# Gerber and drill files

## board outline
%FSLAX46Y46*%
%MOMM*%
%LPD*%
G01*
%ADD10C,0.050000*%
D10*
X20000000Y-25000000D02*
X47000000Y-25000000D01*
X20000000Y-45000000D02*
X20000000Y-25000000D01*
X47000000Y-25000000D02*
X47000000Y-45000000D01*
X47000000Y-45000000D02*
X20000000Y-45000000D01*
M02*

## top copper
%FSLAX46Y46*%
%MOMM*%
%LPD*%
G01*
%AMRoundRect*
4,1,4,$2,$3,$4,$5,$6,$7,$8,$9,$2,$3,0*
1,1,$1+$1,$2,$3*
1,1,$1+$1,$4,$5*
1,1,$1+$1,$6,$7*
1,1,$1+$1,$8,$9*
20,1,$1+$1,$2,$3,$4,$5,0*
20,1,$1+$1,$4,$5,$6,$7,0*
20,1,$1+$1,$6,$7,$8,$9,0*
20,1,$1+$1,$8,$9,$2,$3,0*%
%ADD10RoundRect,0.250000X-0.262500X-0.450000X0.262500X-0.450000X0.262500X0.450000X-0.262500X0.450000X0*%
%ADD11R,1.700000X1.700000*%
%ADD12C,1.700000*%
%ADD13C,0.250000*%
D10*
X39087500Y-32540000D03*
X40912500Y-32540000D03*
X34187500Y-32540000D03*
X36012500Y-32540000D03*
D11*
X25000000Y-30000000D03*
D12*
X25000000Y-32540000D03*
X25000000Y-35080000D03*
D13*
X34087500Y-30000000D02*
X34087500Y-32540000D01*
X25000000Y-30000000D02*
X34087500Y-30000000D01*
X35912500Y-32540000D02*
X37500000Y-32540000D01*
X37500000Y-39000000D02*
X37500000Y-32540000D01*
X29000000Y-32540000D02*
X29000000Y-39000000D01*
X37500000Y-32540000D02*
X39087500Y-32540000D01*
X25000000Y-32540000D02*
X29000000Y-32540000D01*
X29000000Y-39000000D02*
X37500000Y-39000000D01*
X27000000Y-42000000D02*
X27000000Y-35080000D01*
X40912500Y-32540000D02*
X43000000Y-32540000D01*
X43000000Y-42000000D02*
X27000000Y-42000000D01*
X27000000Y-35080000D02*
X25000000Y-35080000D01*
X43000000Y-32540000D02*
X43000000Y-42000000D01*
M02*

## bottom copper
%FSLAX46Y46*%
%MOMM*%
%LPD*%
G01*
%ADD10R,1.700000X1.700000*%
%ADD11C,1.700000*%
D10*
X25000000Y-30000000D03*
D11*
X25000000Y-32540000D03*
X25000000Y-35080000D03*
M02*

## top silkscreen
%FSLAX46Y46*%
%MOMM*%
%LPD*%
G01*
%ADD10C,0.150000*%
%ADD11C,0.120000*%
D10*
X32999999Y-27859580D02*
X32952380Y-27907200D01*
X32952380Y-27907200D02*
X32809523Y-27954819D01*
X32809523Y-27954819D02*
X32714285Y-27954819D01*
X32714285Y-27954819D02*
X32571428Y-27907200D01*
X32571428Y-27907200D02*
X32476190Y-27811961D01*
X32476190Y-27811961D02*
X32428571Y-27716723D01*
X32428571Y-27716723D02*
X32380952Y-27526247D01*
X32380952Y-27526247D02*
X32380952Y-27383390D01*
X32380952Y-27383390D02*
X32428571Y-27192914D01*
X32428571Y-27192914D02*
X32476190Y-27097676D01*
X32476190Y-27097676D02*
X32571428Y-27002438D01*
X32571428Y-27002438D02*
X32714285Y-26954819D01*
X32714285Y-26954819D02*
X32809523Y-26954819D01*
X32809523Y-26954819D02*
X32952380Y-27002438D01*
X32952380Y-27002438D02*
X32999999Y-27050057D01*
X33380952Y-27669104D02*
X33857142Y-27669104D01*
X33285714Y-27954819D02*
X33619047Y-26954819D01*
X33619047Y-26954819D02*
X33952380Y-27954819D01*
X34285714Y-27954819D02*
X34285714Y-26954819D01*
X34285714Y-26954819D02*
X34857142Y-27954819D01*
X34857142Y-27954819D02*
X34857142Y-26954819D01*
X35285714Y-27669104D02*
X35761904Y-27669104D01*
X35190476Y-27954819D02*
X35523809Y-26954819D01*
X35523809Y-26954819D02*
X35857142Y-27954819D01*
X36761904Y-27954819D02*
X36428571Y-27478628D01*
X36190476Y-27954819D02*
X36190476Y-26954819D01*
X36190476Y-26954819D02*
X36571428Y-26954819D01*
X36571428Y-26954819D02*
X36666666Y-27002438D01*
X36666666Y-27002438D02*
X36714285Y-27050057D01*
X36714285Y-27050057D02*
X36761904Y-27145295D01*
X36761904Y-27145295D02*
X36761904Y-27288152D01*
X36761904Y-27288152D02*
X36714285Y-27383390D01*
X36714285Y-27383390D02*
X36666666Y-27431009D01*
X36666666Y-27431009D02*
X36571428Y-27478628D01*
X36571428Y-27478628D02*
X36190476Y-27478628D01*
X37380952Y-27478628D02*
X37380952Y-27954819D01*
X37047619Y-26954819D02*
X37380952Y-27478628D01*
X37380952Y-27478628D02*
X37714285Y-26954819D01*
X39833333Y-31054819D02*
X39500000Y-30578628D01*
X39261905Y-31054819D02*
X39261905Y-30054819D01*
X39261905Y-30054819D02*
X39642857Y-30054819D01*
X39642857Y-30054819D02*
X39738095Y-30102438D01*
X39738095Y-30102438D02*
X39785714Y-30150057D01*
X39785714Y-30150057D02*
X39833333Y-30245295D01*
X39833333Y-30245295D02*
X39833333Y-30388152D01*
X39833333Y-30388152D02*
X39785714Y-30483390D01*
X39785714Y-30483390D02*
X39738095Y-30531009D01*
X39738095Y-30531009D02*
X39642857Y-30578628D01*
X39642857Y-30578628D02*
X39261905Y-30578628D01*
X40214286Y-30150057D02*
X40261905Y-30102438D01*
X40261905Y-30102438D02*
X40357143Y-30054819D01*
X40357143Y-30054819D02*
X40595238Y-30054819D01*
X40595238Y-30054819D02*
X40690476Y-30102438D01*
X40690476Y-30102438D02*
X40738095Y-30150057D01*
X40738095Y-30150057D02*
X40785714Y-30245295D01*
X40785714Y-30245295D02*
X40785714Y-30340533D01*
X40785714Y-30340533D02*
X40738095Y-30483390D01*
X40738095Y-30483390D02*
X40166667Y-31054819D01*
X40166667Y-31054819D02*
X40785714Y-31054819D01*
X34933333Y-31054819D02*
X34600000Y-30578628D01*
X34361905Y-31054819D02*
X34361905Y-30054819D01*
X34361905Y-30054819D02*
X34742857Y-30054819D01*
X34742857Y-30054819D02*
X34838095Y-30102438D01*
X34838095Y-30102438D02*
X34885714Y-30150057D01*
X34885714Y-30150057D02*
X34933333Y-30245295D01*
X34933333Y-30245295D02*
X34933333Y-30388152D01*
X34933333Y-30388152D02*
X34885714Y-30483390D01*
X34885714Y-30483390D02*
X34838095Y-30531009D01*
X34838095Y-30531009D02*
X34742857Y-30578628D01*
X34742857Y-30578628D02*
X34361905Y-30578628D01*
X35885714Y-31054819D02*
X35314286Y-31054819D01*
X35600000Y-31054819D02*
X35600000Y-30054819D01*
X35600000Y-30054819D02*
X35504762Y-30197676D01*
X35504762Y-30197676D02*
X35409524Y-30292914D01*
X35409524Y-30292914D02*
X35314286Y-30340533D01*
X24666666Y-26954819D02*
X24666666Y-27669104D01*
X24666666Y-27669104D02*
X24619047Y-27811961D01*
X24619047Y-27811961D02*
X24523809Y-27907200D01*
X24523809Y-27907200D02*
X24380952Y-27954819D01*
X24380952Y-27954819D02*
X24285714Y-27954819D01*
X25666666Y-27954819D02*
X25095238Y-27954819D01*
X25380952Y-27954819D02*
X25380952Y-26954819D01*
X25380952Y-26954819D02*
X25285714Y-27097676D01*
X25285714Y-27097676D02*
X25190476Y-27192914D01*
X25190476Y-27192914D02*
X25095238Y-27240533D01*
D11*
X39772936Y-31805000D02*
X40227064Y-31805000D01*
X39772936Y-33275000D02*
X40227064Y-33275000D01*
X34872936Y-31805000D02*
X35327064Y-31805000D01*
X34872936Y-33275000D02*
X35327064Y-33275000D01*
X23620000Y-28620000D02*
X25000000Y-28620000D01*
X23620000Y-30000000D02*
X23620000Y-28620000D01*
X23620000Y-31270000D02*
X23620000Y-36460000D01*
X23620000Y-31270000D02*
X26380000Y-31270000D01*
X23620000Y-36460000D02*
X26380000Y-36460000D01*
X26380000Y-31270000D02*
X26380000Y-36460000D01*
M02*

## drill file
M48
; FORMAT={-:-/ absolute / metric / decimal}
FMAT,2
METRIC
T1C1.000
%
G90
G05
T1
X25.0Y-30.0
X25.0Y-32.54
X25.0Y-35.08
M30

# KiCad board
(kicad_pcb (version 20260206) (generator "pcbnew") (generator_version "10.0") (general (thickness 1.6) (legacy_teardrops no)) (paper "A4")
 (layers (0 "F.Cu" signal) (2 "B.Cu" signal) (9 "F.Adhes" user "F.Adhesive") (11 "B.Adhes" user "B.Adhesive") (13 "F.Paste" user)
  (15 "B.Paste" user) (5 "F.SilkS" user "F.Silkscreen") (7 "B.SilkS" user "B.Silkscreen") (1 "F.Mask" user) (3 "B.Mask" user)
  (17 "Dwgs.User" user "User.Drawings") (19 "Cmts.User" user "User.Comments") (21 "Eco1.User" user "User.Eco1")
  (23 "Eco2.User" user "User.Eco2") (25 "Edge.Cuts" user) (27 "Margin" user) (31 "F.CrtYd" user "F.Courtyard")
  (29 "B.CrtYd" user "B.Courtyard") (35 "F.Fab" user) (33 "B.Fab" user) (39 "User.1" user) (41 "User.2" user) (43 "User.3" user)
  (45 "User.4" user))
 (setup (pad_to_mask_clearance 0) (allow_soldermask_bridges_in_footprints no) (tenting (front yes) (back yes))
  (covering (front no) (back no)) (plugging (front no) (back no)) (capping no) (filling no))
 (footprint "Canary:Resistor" (layer "F.Cu") (at 40 32.54)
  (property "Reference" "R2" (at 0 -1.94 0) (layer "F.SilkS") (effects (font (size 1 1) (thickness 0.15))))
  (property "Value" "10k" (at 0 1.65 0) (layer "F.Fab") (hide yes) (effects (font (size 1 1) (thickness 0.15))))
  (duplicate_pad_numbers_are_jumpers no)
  (fp_line (start -0.227064 -0.735) (end 0.227064 -0.735) (stroke (width 0.12) (type solid)) (layer "F.SilkS"))
  (fp_line (start -0.227064 0.735) (end 0.227064 0.735) (stroke (width 0.12) (type solid)) (layer "F.SilkS"))
  (pad "1" smd roundrect (at -0.9125 0) (size 1.025 1.4) (layers "F.Cu" "F.Mask" "F.Paste") (roundrect_rratio 0.243902) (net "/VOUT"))
  (pad "2" smd roundrect (at 0.9125 0) (size 1.025 1.4) (layers "F.Cu" "F.Mask" "F.Paste") (roundrect_rratio 0.243902) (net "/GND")))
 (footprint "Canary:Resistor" (layer "F.Cu") (at 35.1 32.54)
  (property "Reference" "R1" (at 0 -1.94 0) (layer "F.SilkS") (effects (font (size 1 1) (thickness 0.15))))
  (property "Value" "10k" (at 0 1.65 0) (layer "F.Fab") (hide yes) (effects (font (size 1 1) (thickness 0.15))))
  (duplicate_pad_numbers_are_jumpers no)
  (fp_line (start -0.227064 -0.735) (end 0.227064 -0.735) (stroke (width 0.12) (type solid)) (layer "F.SilkS"))
  (fp_line (start -0.227064 0.735) (end 0.227064 0.735) (stroke (width 0.12) (type solid)) (layer "F.SilkS"))
  (pad "1" smd roundrect (at -0.9125 0) (size 1.025 1.4) (layers "F.Cu" "F.Mask" "F.Paste") (roundrect_rratio 0.243902) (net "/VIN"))
  (pad "2" smd roundrect (at 0.9125 0) (size 1.025 1.4) (layers "F.Cu" "F.Mask" "F.Paste") (roundrect_rratio 0.243902) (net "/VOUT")))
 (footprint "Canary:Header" (layer "F.Cu") (at 25 30)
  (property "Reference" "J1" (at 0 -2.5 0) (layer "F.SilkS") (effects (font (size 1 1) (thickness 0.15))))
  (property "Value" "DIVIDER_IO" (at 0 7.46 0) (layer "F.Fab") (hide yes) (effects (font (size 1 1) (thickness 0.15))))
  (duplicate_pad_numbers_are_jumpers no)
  (fp_line (start -1.38 -1.38) (end 0 -1.38) (stroke (width 0.12) (type solid)) (layer "F.SilkS"))
  (fp_line (start -1.38 0) (end -1.38 -1.38) (stroke (width 0.12) (type solid)) (layer "F.SilkS"))
  (fp_line (start -1.38 1.27) (end -1.38 6.46) (stroke (width 0.12) (type solid)) (layer "F.SilkS"))
  (fp_line (start -1.38 1.27) (end 1.38 1.27) (stroke (width 0.12) (type solid)) (layer "F.SilkS"))
  (fp_line (start -1.38 6.46) (end 1.38 6.46) (stroke (width 0.12) (type solid)) (layer "F.SilkS"))
  (fp_line (start 1.38 1.27) (end 1.38 6.46) (stroke (width 0.12) (type solid)) (layer "F.SilkS"))
  (pad "1" thru_hole rect (at 0 0) (size 1.7 1.7) (drill 1) (layers "*.Cu" "*.Mask") (remove_unused_layers no) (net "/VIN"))
  (pad "2" thru_hole circle (at 0 2.54) (size 1.7 1.7) (drill 1) (layers "*.Cu" "*.Mask") (remove_unused_layers no) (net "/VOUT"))
  (pad "3" thru_hole circle (at 0 5.08) (size 1.7 1.7) (drill 1) (layers "*.Cu" "*.Mask") (remove_unused_layers no) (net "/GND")))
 (gr_line (start 20 25) (end 47 25) (stroke (width 0.05) (type default)) (layer "Edge.Cuts"))
 (gr_line (start 20 45) (end 20 25) (stroke (width 0.05) (type default)) (layer "Edge.Cuts"))
 (gr_line (start 47 25) (end 47 45) (stroke (width 0.05) (type default)) (layer "Edge.Cuts"))
 (gr_line (start 47 45) (end 20 45) (stroke (width 0.05) (type default)) (layer "Edge.Cuts"))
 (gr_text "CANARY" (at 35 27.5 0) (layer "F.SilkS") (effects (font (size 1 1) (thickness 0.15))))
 (segment (start 34.0875 30) (end 34.0875 32.54) (width 0.25) (layer "F.Cu") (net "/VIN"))
 (segment (start 25 30) (end 34.0875 30) (width 0.25) (layer "F.Cu") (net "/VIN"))
 (segment (start 35.9125 32.54) (end 37.5 32.54) (width 0.25) (layer "F.Cu") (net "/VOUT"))
 (segment (start 37.5 39) (end 37.5 32.54) (width 0.25) (layer "F.Cu") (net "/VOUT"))
 (segment (start 29 32.54) (end 29 39) (width 0.25) (layer "F.Cu") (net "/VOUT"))
 (segment (start 37.5 32.54) (end 39.0875 32.54) (width 0.25) (layer "F.Cu") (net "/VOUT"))
 (segment (start 25 32.54) (end 29 32.54) (width 0.25) (layer "F.Cu") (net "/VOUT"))
 (segment (start 29 39) (end 37.5 39) (width 0.25) (layer "F.Cu") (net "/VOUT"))
 (segment (start 27 42) (end 27 35.08) (width 0.25) (layer "F.Cu") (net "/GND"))
 (segment (start 40.9125 32.54) (end 43 32.54) (width 0.25) (layer "F.Cu") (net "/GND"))
 (segment (start 43 42) (end 27 42) (width 0.25) (layer "F.Cu") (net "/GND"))
 (segment (start 27 35.08) (end 25 35.08) (width 0.25) (layer "F.Cu") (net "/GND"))
 (segment (start 43 32.54) (end 43 42) (width 0.25) (layer "F.Cu") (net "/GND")))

